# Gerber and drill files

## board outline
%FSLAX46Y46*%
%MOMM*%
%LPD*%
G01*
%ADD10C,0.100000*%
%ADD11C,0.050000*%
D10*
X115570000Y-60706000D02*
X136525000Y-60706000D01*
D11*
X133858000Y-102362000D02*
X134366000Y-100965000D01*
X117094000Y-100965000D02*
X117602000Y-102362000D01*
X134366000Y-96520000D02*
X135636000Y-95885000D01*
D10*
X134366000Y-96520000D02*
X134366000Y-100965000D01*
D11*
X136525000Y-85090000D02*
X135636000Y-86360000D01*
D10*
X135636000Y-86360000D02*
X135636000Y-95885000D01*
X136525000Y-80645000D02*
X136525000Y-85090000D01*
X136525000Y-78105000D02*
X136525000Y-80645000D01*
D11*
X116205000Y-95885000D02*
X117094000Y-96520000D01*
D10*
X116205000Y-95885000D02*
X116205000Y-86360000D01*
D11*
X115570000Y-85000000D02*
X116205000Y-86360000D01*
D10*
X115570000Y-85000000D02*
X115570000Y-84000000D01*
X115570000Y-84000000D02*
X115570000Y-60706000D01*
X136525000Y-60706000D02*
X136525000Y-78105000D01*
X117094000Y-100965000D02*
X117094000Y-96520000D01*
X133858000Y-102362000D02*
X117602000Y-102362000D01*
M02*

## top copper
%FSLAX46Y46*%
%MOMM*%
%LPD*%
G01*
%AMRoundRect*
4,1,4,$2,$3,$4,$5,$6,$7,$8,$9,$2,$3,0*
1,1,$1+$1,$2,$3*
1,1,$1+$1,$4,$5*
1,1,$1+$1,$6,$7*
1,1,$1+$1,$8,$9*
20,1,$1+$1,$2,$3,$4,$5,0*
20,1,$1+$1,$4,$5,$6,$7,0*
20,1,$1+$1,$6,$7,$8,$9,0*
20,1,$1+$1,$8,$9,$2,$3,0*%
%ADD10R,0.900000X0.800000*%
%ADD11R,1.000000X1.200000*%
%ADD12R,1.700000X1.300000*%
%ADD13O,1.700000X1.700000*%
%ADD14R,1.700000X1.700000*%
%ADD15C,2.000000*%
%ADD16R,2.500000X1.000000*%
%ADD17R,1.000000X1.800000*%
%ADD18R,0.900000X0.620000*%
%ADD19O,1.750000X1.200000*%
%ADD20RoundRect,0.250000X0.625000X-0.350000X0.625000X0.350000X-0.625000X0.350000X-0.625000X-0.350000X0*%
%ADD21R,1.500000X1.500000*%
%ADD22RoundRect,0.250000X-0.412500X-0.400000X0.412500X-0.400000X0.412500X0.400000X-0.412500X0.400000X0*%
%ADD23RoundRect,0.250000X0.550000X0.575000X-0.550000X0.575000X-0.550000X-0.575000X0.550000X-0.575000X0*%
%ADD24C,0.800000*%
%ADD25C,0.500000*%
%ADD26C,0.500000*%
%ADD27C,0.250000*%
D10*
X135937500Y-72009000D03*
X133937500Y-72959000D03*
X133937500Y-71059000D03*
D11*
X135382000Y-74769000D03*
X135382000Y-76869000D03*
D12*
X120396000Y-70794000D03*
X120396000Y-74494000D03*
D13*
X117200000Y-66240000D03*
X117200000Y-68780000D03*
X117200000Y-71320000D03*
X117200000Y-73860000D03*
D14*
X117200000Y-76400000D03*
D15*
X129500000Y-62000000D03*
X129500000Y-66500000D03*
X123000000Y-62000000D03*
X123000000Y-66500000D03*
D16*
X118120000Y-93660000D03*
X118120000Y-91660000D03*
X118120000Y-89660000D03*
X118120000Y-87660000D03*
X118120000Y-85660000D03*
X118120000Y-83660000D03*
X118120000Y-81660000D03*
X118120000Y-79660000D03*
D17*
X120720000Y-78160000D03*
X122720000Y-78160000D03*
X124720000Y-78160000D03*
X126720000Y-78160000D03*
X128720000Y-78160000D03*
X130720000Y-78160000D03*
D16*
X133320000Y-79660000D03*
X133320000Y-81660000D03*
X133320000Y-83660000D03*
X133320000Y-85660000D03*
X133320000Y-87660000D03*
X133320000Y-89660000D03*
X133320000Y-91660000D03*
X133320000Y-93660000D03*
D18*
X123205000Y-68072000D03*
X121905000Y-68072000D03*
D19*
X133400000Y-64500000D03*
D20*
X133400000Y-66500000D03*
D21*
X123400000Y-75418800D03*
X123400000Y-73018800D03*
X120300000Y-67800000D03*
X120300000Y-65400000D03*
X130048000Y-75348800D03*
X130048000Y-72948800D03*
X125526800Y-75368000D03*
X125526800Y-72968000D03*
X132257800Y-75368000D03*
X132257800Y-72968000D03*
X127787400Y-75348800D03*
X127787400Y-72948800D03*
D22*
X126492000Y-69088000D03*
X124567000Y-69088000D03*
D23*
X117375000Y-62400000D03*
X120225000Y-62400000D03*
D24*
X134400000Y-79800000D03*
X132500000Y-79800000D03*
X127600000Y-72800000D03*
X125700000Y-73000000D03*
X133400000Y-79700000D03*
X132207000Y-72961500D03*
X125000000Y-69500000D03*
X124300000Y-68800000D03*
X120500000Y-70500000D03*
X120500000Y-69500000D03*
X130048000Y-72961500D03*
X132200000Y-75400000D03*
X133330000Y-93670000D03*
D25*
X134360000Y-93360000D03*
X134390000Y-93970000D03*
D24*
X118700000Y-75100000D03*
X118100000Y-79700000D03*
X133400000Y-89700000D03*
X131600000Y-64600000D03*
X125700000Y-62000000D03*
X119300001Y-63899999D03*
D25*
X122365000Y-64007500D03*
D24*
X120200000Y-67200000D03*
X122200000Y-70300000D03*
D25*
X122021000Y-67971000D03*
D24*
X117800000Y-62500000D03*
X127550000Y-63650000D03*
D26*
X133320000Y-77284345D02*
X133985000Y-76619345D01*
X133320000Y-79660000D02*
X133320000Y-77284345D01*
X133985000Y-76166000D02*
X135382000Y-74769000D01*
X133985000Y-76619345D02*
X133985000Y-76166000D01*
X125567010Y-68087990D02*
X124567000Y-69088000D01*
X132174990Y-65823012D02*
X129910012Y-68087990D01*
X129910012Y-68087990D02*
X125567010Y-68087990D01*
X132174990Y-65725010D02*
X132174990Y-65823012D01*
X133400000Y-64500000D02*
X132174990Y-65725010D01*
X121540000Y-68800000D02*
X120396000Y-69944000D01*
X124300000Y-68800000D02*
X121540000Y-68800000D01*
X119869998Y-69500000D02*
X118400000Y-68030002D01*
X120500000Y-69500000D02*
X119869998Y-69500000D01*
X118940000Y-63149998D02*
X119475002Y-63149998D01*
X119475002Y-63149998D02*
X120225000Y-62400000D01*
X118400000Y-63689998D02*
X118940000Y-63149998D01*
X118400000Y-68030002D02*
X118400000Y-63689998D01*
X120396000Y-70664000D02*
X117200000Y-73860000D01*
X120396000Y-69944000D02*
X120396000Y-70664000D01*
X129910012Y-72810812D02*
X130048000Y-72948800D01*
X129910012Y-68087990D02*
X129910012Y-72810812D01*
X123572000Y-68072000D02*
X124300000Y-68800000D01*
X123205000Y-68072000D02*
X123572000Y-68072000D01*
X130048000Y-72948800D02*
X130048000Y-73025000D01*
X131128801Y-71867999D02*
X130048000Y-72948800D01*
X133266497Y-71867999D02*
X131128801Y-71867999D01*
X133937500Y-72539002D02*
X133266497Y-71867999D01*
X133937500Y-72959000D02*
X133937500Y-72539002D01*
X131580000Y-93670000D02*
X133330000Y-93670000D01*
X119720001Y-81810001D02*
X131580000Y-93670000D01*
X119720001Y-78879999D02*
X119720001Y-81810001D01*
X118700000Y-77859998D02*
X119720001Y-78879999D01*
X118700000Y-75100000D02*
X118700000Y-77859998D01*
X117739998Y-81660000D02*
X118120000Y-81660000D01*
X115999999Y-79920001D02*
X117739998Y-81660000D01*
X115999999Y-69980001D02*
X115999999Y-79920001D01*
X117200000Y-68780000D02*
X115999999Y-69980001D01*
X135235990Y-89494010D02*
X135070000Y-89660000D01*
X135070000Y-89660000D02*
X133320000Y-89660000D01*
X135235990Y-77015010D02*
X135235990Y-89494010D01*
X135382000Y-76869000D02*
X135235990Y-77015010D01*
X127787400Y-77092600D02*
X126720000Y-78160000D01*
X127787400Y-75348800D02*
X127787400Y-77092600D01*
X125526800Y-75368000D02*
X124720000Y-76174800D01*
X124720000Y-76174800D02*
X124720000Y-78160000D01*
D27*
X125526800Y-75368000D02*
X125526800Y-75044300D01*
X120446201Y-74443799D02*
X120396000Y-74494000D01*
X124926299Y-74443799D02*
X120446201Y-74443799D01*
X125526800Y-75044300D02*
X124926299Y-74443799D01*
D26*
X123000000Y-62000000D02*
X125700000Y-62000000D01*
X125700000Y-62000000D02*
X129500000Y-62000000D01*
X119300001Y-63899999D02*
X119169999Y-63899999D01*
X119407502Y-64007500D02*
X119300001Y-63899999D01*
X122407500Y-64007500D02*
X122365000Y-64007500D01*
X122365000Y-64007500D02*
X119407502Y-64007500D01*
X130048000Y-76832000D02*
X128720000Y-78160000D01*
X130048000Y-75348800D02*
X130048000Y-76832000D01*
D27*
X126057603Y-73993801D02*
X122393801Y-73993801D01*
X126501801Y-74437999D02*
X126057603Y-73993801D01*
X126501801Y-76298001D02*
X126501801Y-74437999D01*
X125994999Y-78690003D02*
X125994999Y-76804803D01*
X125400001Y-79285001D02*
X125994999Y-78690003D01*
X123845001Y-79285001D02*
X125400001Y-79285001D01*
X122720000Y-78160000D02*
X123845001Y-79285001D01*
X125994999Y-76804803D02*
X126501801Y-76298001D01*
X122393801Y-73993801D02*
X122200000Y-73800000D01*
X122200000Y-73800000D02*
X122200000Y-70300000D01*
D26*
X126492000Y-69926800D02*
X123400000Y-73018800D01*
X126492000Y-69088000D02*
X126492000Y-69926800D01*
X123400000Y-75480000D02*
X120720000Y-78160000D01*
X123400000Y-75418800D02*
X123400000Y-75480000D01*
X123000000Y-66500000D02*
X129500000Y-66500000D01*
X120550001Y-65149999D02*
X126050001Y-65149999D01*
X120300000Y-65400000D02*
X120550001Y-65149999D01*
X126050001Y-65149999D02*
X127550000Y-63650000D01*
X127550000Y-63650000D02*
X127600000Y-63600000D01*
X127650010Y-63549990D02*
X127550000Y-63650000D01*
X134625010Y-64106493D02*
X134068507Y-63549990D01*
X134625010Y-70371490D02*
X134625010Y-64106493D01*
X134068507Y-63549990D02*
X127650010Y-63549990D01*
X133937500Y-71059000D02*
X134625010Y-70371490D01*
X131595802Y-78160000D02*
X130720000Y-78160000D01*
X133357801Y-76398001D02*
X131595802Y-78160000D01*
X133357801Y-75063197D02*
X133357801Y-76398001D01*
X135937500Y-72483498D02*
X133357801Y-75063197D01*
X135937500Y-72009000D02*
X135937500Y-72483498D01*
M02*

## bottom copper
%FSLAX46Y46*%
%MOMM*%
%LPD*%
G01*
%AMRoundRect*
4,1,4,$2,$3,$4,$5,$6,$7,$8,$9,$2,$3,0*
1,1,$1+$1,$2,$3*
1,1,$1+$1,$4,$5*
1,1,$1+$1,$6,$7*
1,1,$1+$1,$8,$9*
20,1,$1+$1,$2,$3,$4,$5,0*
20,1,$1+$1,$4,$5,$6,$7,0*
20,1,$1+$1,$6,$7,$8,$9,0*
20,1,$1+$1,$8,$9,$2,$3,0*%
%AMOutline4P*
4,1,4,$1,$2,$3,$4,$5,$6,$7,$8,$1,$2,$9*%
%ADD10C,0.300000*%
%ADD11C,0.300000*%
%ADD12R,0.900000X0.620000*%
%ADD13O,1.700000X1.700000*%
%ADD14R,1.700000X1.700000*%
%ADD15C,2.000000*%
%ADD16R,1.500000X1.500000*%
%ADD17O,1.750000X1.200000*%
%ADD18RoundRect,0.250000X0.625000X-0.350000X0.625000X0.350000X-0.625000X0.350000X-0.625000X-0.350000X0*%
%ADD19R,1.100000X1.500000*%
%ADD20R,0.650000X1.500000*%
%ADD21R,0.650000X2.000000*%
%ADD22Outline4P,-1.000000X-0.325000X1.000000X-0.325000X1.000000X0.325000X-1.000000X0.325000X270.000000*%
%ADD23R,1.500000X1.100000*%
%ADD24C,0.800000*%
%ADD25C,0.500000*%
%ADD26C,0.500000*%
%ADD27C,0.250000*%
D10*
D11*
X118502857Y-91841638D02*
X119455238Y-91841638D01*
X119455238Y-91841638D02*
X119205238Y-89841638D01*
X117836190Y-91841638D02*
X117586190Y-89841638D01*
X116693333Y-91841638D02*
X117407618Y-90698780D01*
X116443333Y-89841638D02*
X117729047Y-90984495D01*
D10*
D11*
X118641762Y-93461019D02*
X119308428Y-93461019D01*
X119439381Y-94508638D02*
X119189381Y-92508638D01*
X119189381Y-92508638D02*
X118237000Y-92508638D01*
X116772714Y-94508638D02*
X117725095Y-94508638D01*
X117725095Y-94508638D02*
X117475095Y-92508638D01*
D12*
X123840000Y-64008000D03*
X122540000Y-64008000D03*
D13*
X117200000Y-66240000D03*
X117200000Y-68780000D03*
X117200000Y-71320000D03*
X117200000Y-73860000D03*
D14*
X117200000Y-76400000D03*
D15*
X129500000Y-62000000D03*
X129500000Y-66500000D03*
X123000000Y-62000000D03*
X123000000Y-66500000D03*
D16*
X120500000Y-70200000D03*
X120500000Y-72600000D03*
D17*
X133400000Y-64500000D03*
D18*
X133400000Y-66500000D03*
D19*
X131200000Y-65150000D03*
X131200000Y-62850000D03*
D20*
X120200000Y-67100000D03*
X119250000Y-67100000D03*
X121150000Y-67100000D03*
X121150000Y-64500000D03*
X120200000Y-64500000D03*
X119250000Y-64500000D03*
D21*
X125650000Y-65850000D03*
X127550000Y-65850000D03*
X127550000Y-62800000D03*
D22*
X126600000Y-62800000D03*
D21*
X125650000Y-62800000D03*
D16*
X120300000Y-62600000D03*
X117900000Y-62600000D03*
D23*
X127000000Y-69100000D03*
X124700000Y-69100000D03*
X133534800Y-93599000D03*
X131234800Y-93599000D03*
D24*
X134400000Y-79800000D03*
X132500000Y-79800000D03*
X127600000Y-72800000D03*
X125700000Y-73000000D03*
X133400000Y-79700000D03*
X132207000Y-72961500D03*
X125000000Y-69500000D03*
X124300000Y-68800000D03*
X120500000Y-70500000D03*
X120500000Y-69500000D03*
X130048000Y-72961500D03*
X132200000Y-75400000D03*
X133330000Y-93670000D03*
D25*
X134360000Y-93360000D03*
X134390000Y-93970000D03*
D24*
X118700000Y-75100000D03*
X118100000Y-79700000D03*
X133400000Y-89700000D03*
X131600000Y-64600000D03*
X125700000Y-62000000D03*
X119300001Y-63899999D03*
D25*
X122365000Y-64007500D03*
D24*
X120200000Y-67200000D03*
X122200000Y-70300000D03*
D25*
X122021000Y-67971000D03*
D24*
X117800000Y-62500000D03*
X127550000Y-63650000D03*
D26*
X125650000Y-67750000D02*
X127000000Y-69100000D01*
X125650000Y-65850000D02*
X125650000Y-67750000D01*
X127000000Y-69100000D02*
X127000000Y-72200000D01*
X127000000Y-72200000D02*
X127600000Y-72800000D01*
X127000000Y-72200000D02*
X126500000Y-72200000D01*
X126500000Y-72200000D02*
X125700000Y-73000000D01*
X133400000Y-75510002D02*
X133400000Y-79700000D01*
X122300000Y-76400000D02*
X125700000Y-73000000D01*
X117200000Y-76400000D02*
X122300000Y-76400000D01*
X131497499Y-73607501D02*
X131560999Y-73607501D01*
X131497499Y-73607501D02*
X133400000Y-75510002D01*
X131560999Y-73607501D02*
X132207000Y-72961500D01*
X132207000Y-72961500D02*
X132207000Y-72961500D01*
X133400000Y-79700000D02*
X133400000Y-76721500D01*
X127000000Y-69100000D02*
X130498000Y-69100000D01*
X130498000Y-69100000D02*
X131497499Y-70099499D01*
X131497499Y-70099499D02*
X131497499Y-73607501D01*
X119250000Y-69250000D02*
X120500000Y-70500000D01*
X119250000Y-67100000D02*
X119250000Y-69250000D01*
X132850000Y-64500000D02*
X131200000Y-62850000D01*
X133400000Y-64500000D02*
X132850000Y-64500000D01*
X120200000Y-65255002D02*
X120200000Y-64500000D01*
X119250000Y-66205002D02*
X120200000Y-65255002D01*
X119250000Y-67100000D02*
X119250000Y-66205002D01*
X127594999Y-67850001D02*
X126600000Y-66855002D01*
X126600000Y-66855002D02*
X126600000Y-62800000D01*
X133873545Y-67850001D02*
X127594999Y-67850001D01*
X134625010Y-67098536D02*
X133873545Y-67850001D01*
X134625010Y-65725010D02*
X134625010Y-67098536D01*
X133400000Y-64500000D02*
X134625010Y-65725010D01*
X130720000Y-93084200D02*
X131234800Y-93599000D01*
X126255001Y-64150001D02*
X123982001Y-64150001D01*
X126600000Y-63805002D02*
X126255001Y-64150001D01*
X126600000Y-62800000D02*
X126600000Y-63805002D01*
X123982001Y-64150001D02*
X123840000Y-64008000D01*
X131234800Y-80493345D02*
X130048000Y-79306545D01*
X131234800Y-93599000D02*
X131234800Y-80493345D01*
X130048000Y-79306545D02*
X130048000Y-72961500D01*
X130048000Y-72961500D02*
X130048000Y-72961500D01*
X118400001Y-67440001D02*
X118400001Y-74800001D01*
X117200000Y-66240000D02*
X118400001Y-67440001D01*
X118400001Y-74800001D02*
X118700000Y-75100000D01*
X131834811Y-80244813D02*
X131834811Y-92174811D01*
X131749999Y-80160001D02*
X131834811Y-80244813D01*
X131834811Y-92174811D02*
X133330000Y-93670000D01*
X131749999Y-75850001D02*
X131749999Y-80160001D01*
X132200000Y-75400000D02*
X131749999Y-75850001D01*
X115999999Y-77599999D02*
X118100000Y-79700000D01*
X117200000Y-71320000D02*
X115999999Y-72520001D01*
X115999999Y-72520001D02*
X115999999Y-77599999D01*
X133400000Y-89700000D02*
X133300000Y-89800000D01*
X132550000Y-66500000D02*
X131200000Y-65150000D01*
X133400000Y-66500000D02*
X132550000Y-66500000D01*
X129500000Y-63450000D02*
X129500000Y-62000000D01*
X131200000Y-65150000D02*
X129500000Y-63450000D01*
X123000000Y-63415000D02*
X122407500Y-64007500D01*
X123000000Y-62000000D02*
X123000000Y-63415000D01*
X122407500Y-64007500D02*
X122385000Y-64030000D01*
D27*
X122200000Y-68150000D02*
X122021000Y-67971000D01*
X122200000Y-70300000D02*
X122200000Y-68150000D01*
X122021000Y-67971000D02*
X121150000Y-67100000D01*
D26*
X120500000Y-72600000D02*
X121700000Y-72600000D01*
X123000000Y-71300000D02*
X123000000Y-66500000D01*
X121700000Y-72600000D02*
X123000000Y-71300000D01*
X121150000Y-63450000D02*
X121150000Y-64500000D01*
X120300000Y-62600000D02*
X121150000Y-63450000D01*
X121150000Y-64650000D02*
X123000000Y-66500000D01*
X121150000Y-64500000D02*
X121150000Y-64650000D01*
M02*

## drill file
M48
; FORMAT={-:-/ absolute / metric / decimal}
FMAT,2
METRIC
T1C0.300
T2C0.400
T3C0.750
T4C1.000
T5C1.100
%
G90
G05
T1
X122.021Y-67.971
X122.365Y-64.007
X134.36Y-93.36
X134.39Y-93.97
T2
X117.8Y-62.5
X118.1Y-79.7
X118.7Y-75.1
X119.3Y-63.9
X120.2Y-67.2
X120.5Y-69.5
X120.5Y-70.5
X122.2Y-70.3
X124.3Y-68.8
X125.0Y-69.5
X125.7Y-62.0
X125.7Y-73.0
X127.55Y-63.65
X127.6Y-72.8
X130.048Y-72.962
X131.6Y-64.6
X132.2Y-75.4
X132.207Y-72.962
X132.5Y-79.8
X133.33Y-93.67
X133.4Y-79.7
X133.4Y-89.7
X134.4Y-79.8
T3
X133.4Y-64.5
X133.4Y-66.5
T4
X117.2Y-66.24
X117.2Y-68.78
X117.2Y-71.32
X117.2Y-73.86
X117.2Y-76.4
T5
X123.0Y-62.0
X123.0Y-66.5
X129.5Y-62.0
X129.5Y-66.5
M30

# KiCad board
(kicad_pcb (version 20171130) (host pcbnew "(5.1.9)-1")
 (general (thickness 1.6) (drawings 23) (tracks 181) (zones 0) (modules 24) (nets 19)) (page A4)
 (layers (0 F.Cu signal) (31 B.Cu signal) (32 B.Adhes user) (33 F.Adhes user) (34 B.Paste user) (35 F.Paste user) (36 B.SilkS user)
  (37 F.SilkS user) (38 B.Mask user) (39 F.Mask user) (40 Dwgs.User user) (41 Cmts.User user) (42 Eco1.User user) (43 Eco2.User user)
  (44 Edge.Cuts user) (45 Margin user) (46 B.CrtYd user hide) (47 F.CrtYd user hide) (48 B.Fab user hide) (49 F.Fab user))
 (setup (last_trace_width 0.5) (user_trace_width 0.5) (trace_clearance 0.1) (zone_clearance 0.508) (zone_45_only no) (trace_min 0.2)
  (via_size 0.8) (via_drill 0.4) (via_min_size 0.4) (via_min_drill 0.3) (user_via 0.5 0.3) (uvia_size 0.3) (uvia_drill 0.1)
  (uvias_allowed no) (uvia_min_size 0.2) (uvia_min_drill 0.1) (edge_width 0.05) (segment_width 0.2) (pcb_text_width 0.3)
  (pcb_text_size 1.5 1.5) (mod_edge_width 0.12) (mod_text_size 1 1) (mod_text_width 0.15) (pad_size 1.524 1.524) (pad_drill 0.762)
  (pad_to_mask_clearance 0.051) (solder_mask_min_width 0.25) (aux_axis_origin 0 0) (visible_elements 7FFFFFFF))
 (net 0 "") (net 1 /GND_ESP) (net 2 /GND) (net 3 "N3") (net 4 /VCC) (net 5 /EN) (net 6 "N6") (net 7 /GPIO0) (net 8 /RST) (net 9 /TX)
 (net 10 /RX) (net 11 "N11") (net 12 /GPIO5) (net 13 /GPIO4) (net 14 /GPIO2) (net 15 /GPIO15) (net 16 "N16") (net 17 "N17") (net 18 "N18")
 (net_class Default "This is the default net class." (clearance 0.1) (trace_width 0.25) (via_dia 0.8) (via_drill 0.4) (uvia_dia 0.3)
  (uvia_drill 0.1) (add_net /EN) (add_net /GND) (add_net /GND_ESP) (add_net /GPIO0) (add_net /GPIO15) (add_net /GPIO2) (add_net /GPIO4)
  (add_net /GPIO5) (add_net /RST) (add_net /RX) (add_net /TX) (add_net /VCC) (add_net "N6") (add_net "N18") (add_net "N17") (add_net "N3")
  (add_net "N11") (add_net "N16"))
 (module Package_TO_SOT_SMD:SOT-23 (layer F.Cu) (at 134.9375 72.009)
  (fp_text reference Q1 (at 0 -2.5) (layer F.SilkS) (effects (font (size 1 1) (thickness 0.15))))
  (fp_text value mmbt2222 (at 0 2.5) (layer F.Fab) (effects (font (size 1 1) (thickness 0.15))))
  (pad 3 smd rect (at 1 0) (size 0.9 0.8) (layers F.Cu F.Paste F.Mask) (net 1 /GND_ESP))
  (pad 2 smd rect (at -1 0.95) (size 0.9 0.8) (layers F.Cu F.Paste F.Mask) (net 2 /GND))
  (pad 1 smd rect (at -1 -0.95) (size 0.9 0.8) (layers F.Cu F.Paste F.Mask) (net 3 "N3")))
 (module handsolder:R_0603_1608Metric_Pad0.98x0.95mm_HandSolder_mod (layer F.Cu) (at 135.382 75.819 90)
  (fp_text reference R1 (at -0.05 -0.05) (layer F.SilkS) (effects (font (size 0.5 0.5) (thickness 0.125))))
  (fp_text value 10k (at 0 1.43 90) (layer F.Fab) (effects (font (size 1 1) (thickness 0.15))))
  (pad 2 smd rect (at 1.05 0 90) (size 1.2 1) (layers F.Cu F.Paste F.Mask) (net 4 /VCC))
  (pad 1 smd rect (at -1.05 0 90) (size 1.2 1) (layers F.Cu F.Paste F.Mask) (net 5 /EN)))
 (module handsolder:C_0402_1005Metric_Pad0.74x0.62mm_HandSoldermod (layer B.Cu) (at 123.19 64.008)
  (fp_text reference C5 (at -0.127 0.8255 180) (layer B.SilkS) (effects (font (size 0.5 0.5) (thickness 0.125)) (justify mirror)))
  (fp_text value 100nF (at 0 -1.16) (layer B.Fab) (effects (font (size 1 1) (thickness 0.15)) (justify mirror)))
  (pad 2 smd rect (at 0.65 0) (size 0.9 0.62) (layers B.Cu B.Paste B.Mask) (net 2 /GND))
  (pad 1 smd rect (at -0.65 0) (size 0.9 0.62) (layers B.Cu B.Paste B.Mask) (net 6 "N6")))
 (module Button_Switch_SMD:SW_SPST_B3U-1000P (layer F.Cu) (at 120.396 72.644 90)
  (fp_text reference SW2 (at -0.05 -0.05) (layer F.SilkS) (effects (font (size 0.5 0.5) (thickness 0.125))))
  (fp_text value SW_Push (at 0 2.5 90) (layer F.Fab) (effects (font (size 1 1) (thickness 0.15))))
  (pad 2 smd rect (at 1.85 0 90) (size 1.3 1.7) (layers F.Cu F.Paste F.Mask) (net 2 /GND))
  (pad 1 smd rect (at -1.85 0 90) (size 1.3 1.7) (layers F.Cu F.Paste F.Mask) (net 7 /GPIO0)))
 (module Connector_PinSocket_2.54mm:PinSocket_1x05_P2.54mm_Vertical (layer F.Cu) (at 117.2 76.4 180)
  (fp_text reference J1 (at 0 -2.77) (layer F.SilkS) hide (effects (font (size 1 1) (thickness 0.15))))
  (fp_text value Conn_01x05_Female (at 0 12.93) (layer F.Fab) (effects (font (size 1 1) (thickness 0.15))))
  (pad 5 thru_hole oval (at 0 10.16 180) (size 1.7 1.7) (drill 1) (layers *.Cu *.Mask) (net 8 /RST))
  (pad 4 thru_hole oval (at 0 7.62 180) (size 1.7 1.7) (drill 1) (layers *.Cu *.Mask) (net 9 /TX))
  (pad 3 thru_hole oval (at 0 5.08 180) (size 1.7 1.7) (drill 1) (layers *.Cu *.Mask) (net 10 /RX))
  (pad 2 thru_hole oval (at 0 2.54 180) (size 1.7 1.7) (drill 1) (layers *.Cu *.Mask) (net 2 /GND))
  (pad 1 thru_hole rect (at 0 0 180) (size 1.7 1.7) (drill 1) (layers *.Cu *.Mask) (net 4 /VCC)))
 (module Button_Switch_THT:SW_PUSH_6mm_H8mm (layer F.Cu) (at 123 62)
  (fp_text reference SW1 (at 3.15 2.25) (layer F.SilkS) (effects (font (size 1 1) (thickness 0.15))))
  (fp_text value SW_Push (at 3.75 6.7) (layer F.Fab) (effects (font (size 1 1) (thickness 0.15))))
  (pad 1 thru_hole circle (at 6.5 0 90) (size 2 2) (drill 1.1) (layers *.Cu *.Mask) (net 6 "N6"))
  (pad 2 thru_hole circle (at 6.5 4.5 90) (size 2 2) (drill 1.1) (layers *.Cu *.Mask) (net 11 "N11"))
  (pad 1 thru_hole circle (at 0 0 90) (size 2 2) (drill 1.1) (layers *.Cu *.Mask) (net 6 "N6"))
  (pad 2 thru_hole circle (at 0 4.5 90) (size 2 2) (drill 1.1) (layers *.Cu *.Mask) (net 11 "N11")))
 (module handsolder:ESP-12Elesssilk (layer F.Cu) (at 125.72 90.16 180)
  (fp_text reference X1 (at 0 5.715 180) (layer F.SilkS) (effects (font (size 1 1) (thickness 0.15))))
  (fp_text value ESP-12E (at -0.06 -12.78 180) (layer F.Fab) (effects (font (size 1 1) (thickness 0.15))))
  (pad 22 smd rect (at 7.6 -3.5 180) (size 2.5 1) (layers F.Cu F.Paste F.Mask))
  (pad 21 smd rect (at 7.6 -1.5 180) (size 2.5 1) (layers F.Cu F.Paste F.Mask))
  (pad 20 smd rect (at 7.6 0.5 180) (size 2.5 1) (layers F.Cu F.Paste F.Mask))
  (pad 19 smd rect (at 7.6 2.5 180) (size 2.5 1) (layers F.Cu F.Paste F.Mask))
  (pad 18 smd rect (at 7.6 4.5 180) (size 2.5 1) (layers F.Cu F.Paste F.Mask))
  (pad 17 smd rect (at 7.6 6.5 180) (size 2.5 1) (layers F.Cu F.Paste F.Mask))
  (pad 16 smd rect (at 7.6 8.5 180) (size 2.5 1) (layers F.Cu F.Paste F.Mask) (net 9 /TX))
  (pad 15 smd rect (at 7.6 10.5 180) (size 2.5 1) (layers F.Cu F.Paste F.Mask) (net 10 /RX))
  (pad 14 smd rect (at 5 12 180) (size 1 1.8) (layers F.Cu F.Paste F.Mask) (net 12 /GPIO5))
  (pad 13 smd rect (at 3 12 180) (size 1 1.8) (layers F.Cu F.Paste F.Mask) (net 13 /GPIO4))
  (pad 12 smd rect (at 1 12 180) (size 1 1.8) (layers F.Cu F.Paste F.Mask) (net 7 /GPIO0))
  (pad 11 smd rect (at -1 12 180) (size 1 1.8) (layers F.Cu F.Paste F.Mask) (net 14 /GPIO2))
  (pad 10 smd rect (at -3 12 180) (size 1 1.8) (layers F.Cu F.Paste F.Mask) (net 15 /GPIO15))
  (pad 9 smd rect (at -5 12 180) (size 1 1.8) (layers F.Cu F.Paste F.Mask) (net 1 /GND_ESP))
  (pad 8 smd rect (at -7.6 10.5 180) (size 2.5 1) (layers F.Cu F.Paste F.Mask) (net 4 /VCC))
  (pad 7 smd rect (at -7.6 8.5 180) (size 2.5 1) (layers F.Cu F.Paste F.Mask))
  (pad 6 smd rect (at -7.6 6.5 180) (size 2.5 1) (layers F.Cu F.Paste F.Mask))
  (pad 5 smd rect (at -7.6 4.5 180) (size 2.5 1) (layers F.Cu F.Paste F.Mask))
  (pad 4 smd rect (at -7.6 2.5 180) (size 2.5 1) (layers F.Cu F.Paste F.Mask))
  (pad 3 smd rect (at -7.6 0.5 180) (size 2.5 1) (layers F.Cu F.Paste F.Mask) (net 5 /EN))
  (pad 2 smd rect (at -7.6 -1.5 180) (size 2.5 1) (layers F.Cu F.Paste F.Mask))
  (pad 1 smd rect (at -7.6 -3.5 180) (size 2.5 1) (layers F.Cu F.Paste F.Mask) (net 8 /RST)))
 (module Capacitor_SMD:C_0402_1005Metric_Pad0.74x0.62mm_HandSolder (layer F.Cu) (at 122.555 68.072)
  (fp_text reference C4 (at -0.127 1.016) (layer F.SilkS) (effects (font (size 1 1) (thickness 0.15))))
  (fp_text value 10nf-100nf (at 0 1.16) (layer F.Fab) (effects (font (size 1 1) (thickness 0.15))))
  (pad 2 smd rect (at 0.65 0) (size 0.9 0.62) (layers F.Cu F.Paste F.Mask) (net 2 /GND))
  (pad 1 smd rect (at -0.65 0) (size 0.9 0.62) (layers F.Cu F.Paste F.Mask) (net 13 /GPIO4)))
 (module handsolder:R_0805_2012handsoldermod (layer B.Cu) (at 120.5 71.4 90)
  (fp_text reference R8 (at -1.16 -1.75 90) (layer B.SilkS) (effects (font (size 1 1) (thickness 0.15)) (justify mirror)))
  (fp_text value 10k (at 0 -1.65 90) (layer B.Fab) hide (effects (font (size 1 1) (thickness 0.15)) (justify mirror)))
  (pad 2 smd rect (at 1.2 0 90) (size 1.5 1.5) (layers B.Cu B.Paste B.Mask) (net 2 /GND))
  (pad 1 smd rect (at -1.2 0 90) (size 1.5 1.5) (layers B.Cu B.Paste B.Mask) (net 11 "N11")))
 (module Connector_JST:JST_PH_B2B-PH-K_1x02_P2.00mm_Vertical (layer F.Cu) (at 133.4 66.5 90)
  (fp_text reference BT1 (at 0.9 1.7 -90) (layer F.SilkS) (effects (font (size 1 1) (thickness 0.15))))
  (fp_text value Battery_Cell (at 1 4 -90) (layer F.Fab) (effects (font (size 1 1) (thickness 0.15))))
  (pad 2 thru_hole oval (at 2 0 90) (size 1.2 1.75) (drill 0.75) (layers *.Cu *.Mask) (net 2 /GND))
  (pad 1 thru_hole roundrect (at 0 0 90) (size 1.2 1.75) (drill 0.75) (layers *.Cu *.Mask) (roundrect_rratio 0.208333) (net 6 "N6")))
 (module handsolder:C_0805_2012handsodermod (layer B.Cu) (at 131.2 64 270)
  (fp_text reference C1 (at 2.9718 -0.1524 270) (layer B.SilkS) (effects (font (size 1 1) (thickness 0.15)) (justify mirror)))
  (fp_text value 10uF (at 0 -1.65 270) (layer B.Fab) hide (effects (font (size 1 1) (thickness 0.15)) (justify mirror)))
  (pad 2 smd rect (at 1.15 0 270) (size 1.5 1.1) (layers B.Cu B.Paste B.Mask) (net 6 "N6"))
  (pad 1 smd rect (at -1.15 0 270) (size 1.5 1.1) (layers B.Cu B.Paste B.Mask) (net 2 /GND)))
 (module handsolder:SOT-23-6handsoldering (layer B.Cu) (at 120.2 65.8 270)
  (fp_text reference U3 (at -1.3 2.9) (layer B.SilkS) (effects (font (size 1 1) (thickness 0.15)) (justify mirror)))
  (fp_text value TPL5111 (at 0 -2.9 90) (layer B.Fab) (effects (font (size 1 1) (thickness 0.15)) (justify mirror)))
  (pad 5 smd rect (at 1.3 0 270) (size 1.5 0.65) (layers B.Cu B.Paste B.Mask) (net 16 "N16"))
  (pad 6 smd rect (at 1.3 0.95 270) (size 1.5 0.65) (layers B.Cu B.Paste B.Mask) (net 2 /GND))
  (pad 4 smd rect (at 1.3 -0.95 270) (size 1.5 0.65) (layers B.Cu B.Paste B.Mask) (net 13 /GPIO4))
  (pad 3 smd rect (at -1.3 -0.95 270) (size 1.5 0.65) (layers B.Cu B.Paste B.Mask) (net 11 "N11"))
  (pad 2 smd rect (at -1.3 0 270) (size 1.5 0.65) (layers B.Cu B.Paste B.Mask) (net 2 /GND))
  (pad 1 smd rect (at -1.3 0.95 270) (size 1.5 0.65) (layers B.Cu B.Paste B.Mask) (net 6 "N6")))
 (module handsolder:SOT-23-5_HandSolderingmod (layer B.Cu) (at 126.6 64.35 270)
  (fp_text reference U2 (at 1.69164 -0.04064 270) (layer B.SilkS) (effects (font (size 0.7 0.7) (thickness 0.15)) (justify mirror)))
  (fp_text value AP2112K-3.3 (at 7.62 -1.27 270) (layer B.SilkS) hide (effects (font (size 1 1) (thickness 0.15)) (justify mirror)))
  (pad 5 smd rect (at 1.5 0.95 270) (size 2 0.65) (layers B.Cu B.Paste B.Mask) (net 4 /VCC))
  (pad 4 smd rect (at 1.5 -0.95 270) (size 2 0.65) (layers B.Cu B.Paste B.Mask))
  (pad 3 smd rect (at -1.55 -0.95 270) (size 2 0.65) (layers B.Cu B.Paste B.Mask) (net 3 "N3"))
  (pad 2 smd trapezoid (at -1.55 0 270) (size 2 0.65) (layers B.Cu B.Paste B.Mask) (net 2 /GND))
  (pad 1 smd rect (at -1.55 0.95 270) (size 2 0.65) (layers B.Cu B.Paste B.Mask) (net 6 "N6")))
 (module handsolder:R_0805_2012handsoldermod (layer F.Cu) (at 123.4 74.2188 270)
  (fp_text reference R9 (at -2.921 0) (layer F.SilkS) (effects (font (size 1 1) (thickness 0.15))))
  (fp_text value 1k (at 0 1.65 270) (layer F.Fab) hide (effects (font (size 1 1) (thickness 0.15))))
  (pad 2 smd rect (at 1.2 0 270) (size 1.5 1.5) (layers F.Cu F.Paste F.Mask) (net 12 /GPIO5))
  (pad 1 smd rect (at -1.2 0 270) (size 1.5 1.5) (layers F.Cu F.Paste F.Mask) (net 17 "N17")))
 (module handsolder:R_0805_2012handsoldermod (layer F.Cu) (at 120.3 66.6 270)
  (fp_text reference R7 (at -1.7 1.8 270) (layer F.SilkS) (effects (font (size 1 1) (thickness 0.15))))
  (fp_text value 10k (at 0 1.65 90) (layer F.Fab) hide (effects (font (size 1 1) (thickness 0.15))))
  (pad 2 smd rect (at 1.2 0 270) (size 1.5 1.5) (layers F.Cu F.Paste F.Mask) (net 16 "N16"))
  (pad 1 smd rect (at -1.2 0 270) (size 1.5 1.5) (layers F.Cu F.Paste F.Mask) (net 3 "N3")))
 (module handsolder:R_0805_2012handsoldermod (layer B.Cu) (at 119.1 62.6)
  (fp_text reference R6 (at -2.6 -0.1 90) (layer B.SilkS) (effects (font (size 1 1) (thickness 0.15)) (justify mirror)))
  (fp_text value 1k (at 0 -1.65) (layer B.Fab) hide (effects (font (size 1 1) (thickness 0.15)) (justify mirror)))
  (pad 2 smd rect (at 1.2 0) (size 1.5 1.5) (layers B.Cu B.Paste B.Mask) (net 11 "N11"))
  (pad 1 smd rect (at -1.2 0) (size 1.5 1.5) (layers B.Cu B.Paste B.Mask) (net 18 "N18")))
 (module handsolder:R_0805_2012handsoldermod (layer F.Cu) (at 130.048 74.1488 270)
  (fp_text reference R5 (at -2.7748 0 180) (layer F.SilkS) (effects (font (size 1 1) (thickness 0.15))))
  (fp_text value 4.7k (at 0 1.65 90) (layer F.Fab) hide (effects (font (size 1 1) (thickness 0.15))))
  (pad 2 smd rect (at 1.2 0 270) (size 1.5 1.5) (layers F.Cu F.Paste F.Mask) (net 15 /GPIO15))
  (pad 1 smd rect (at -1.2 0 270) (size 1.5 1.5) (layers F.Cu F.Paste F.Mask) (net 2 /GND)))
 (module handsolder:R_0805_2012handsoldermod (layer F.Cu) (at 125.5268 74.168 270)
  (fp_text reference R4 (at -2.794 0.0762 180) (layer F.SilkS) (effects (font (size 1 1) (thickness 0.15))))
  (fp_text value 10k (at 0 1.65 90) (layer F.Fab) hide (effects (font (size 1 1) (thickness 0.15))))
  (pad 2 smd rect (at 1.2 0 270) (size 1.5 1.5) (layers F.Cu F.Paste F.Mask) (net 7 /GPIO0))
  (pad 1 smd rect (at -1.2 0 270) (size 1.5 1.5) (layers F.Cu F.Paste F.Mask) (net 4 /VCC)))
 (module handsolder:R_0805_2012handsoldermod (layer F.Cu) (at 132.2578 74.168 270)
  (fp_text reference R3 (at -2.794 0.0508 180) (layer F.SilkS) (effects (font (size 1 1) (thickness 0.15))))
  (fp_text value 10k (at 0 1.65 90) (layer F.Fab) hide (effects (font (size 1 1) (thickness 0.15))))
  (pad 2 smd rect (at 1.2 0 270) (size 1.5 1.5) (layers F.Cu F.Paste F.Mask) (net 8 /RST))
  (pad 1 smd rect (at -1.2 0 270) (size 1.5 1.5) (layers F.Cu F.Paste F.Mask) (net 4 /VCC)))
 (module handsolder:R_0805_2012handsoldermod (layer F.Cu) (at 127.7874 74.1488 270)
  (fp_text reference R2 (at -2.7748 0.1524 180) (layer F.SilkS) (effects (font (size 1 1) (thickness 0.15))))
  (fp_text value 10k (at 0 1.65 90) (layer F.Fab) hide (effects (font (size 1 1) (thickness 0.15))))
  (pad 2 smd rect (at 1.2 0 270) (size 1.5 1.5) (layers F.Cu F.Paste F.Mask) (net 14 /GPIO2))
  (pad 1 smd rect (at -1.2 0 270) (size 1.5 1.5) (layers F.Cu F.Paste F.Mask) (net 4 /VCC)))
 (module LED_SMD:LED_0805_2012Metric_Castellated (layer F.Cu) (at 125.5295 69.088)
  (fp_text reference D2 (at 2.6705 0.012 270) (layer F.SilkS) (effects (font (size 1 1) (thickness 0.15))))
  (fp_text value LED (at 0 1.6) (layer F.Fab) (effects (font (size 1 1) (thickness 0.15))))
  (pad 2 smd roundrect (at 0.9625 0) (size 1.325 1.3) (layers F.Cu F.Paste F.Mask) (roundrect_rratio 0.1923076923076923) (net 17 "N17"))
  (pad 1 smd roundrect (at -0.9625 0) (size 1.325 1.3) (layers F.Cu F.Paste F.Mask) (roundrect_rratio 0.1923076923076923) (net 2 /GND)))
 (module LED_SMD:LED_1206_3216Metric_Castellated (layer F.Cu) (at 118.8 62.4 180)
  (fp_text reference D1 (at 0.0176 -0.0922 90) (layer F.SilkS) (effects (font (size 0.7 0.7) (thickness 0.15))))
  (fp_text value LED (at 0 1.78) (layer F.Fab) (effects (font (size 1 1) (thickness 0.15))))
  (pad 2 smd roundrect (at 1.425 0 180) (size 1.6 1.65) (layers F.Cu F.Paste F.Mask) (roundrect_rratio 0.15625) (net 18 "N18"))
  (pad 1 smd roundrect (at -1.425 0 180) (size 1.6 1.65) (layers F.Cu F.Paste F.Mask) (roundrect_rratio 0.15625) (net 2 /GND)))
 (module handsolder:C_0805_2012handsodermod (layer B.Cu) (at 125.85 69.1)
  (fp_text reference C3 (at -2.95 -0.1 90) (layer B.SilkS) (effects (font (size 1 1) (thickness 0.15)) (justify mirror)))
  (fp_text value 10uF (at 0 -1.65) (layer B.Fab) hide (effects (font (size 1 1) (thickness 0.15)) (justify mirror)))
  (pad 2 smd rect (at 1.15 0) (size 1.5 1.1) (layers B.Cu B.Paste B.Mask) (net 4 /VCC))
  (pad 1 smd rect (at -1.15 0) (size 1.5 1.1) (layers B.Cu B.Paste B.Mask) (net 2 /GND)))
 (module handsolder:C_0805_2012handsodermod (layer B.Cu) (at 132.3848 93.599)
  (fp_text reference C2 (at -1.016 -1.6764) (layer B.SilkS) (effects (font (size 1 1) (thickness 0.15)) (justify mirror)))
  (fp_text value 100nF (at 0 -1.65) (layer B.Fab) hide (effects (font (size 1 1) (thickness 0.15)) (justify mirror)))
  (pad 2 smd rect (at 1.15 0) (size 1.5 1.1) (layers B.Cu B.Paste B.Mask) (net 8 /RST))
  (pad 1 smd rect (at -1.15 0) (size 1.5 1.1) (layers B.Cu B.Paste B.Mask) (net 2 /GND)))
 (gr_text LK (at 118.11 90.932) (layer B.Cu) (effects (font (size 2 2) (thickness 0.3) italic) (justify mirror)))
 (gr_line (start 115.57 60.706) (end 136.525 60.706) (layer Edge.Cuts) (width 0.1))
 (gr_line (start 133.858 102.362) (end 134.366 100.965) (layer Edge.Cuts) (width 0.05))
 (gr_line (start 117.094 100.965) (end 117.602 102.362) (layer Edge.Cuts) (width 0.05))
 (gr_line (start 134.366 96.52) (end 135.636 95.885) (layer Edge.Cuts) (width 0.05))
 (gr_line (start 134.366 96.52) (end 134.366 100.965) (layer Edge.Cuts) (width 0.1))
 (gr_line (start 136.525 85.09) (end 135.636 86.36) (layer Edge.Cuts) (width 0.05))
 (gr_line (start 135.636 86.36) (end 135.636 95.885) (layer Edge.Cuts) (width 0.1))
 (gr_line (start 136.525 80.645) (end 136.525 85.09) (layer Edge.Cuts) (width 0.1))
 (gr_line (start 136.525 78.105) (end 136.525 80.645) (layer Edge.Cuts) (width 0.1))
 (gr_line (start 116.205 95.885) (end 117.094 96.52) (layer Edge.Cuts) (width 0.05))
 (gr_line (start 116.205 95.885) (end 116.205 86.36) (layer Edge.Cuts) (width 0.1))
 (gr_line (start 115.57 85) (end 116.205 86.36) (layer Edge.Cuts) (width 0.05))
 (gr_line (start 115.57 85) (end 115.57 84) (layer Edge.Cuts) (width 0.1))
 (gr_line (start 115.57 84) (end 115.57 60.706) (layer Edge.Cuts) (width 0.1))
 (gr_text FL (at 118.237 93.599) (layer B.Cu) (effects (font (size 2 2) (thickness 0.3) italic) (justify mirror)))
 (gr_line (start 136.525 60.706) (end 136.525 78.105) (layer Edge.Cuts) (width 0.1))
 (gr_line (start 117.094 100.965) (end 117.094 96.52) (layer Edge.Cuts) (width 0.1))
 (gr_line (start 133.858 102.362) (end 117.602 102.362) (layer Edge.Cuts) (width 0.1))
 (via (at 134.4 79.8) (size 0.8) (drill 0.4) (layers F.Cu B.Cu) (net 4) (status 30))
 (via (at 132.5 79.8) (size 0.8) (drill 0.4) (layers F.Cu B.Cu) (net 4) (status 30))
 (segment (start 125.65 67.75) (end 127 69.1) (width 0.5) (layer B.Cu) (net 4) (status 20))
 (segment (start 125.65 65.85) (end 125.65 67.75) (width 0.5) (layer B.Cu) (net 4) (status 10))
 (segment (start 127 69.1) (end 127 72.2) (width 0.5) (layer B.Cu) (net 4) (status 10))
 (segment (start 127 72.2) (end 127.6 72.8) (width 0.5) (layer B.Cu) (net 4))
 (segment (start 127 72.2) (end 126.5 72.2) (width 0.5) (layer B.Cu) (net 4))
 (segment (start 126.5 72.2) (end 125.7 73) (width 0.5) (layer B.Cu) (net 4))
 (via (at 127.6 72.8) (size 0.8) (drill 0.4) (layers F.Cu B.Cu) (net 4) (status 30))
 (via (at 125.7 73) (size 0.8) (drill 0.4) (layers F.Cu B.Cu) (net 4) (status 30))
 (segment (start 133.4 75.510002) (end 133.4 79.7) (width 0.5) (layer B.Cu) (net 4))
 (via (at 133.4 79.7) (size 0.8) (drill 0.4) (layers F.Cu B.Cu) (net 4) (status 30))
 (segment (start 122.3 76.4) (end 125.7 73) (width 0.5) (layer B.Cu) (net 4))
 (segment (start 117.2 76.4) (end 122.3 76.4) (width 0.5) (layer B.Cu) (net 4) (status 10))
 (segment (start 131.497499 73.607501) (end 131.560999 73.607501) (width 0.5) (layer B.Cu) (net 4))
 (segment (start 131.497499 73.607501) (end 133.4 75.510002) (width 0.5) (layer B.Cu) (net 4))
 (segment (start 131.560999 73.607501) (end 132.207 72.9615) (width 0.5) (layer B.Cu) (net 4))
 (segment (start 132.207 72.9615) (end 132.207 72.9615) (width 0.5) (layer B.Cu) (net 4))
 (via (at 132.207 72.9615) (size 0.8) (drill 0.4) (layers F.Cu B.Cu) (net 4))
 (segment (start 133.4 79.7) (end 133.4 76.7215) (width 0.5) (layer B.Cu) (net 4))
 (segment (start 133.32 77.284345) (end 133.985 76.619345) (width 0.5) (layer F.Cu) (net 4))
 (segment (start 133.32 79.66) (end 133.32 77.284345) (width 0.5) (layer F.Cu) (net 4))
 (segment (start 133.985 76.166) (end 135.382 74.769) (width 0.5) (layer F.Cu) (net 4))
 (segment (start 133.985 76.619345) (end 133.985 76.166) (width 0.5) (layer F.Cu) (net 4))
 (segment (start 127 69.1) (end 130.498 69.1) (width 0.5) (layer B.Cu) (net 4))
 (segment (start 130.498 69.1) (end 131.497499 70.099499) (width 0.5) (layer B.Cu) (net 4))
 (segment (start 131.497499 70.099499) (end 131.497499 73.607501) (width 0.5) (layer B.Cu) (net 4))
 (via (at 125 69.5) (size 0.8) (drill 0.4) (layers F.Cu B.Cu) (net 2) (status 30))
 (via (at 124.3 68.8) (size 0.8) (drill 0.4) (layers F.Cu B.Cu) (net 2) (status 30))
 (via (at 120.5 70.5) (size 0.8) (drill 0.4) (layers F.Cu B.Cu) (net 2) (status 30))
 (via (at 120.5 69.5) (size 0.8) (drill 0.4) (layers F.Cu B.Cu) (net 2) (status 30))
 (segment (start 119.25 69.25) (end 120.5 70.5) (width 0.5) (layer B.Cu) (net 2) (status 20))
 (segment (start 119.25 67.1) (end 119.25 69.25) (width 0.5) (layer B.Cu) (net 2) (status 10))
 (segment (start 132.85 64.5) (end 131.2 62.85) (width 0.5) (layer B.Cu) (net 2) (status 30))
 (segment (start 133.4 64.5) (end 132.85 64.5) (width 0.5) (layer B.Cu) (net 2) (status 30))
 (segment (start 120.2 65.255002) (end 120.2 64.5) (width 0.5) (layer B.Cu) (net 2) (status 20))
 (segment (start 119.25 66.205002) (end 120.2 65.255002) (width 0.5) (layer B.Cu) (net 2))
 (segment (start 119.25 67.1) (end 119.25 66.205002) (width 0.5) (layer B.Cu) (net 2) (status 10))
 (segment (start 127.594999 67.850001) (end 126.6 66.855002) (width 0.5) (layer B.Cu) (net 2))
 (segment (start 126.6 66.855002) (end 126.6 62.8) (width 0.5) (layer B.Cu) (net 2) (status 20))
 (segment (start 133.873545 67.850001) (end 127.594999 67.850001) (width 0.5) (layer B.Cu) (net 2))
 (segment (start 134.62501 67.098536) (end 133.873545 67.850001) (width 0.5) (layer B.Cu) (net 2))
 (segment (start 134.62501 65.72501) (end 134.62501 67.098536) (width 0.5) (layer B.Cu) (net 2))
 (segment (start 133.4 64.5) (end 134.62501 65.72501) (width 0.5) (layer B.Cu) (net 2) (status 10))
 (segment (start 125.56701 68.08799) (end 124.567 69.088) (width 0.5) (layer F.Cu) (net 2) (status 20))
 (segment (start 132.17499 65.823012) (end 129.910012 68.08799) (width 0.5) (layer F.Cu) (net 2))
 (segment (start 129.910012 68.08799) (end 125.56701 68.08799) (width 0.5) (layer F.Cu) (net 2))
 (segment (start 132.17499 65.72501) (end 132.17499 65.823012) (width 0.5) (layer F.Cu) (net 2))
 (segment (start 133.4 64.5) (end 132.17499 65.72501) (width 0.5) (layer F.Cu) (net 2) (status 10))
 (segment (start 121.54 68.8) (end 120.396 69.944) (width 0.5) (layer F.Cu) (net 2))
 (segment (start 124.3 68.8) (end 121.54 68.8) (width 0.5) (layer F.Cu) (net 2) (status 10))
 (segment (start 119.869998 69.5) (end 118.4 68.030002) (width 0.5) (layer F.Cu) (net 2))
 (segment (start 120.5 69.5) (end 119.869998 69.5) (width 0.5) (layer F.Cu) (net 2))
 (segment (start 118.94 63.149998) (end 119.475002 63.149998) (width 0.5) (layer F.Cu) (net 2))
 (segment (start 119.475002 63.149998) (end 120.225 62.4) (width 0.5) (layer F.Cu) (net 2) (status 20))
 (segment (start 118.4 63.689998) (end 118.94 63.149998) (width 0.5) (layer F.Cu) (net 2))
 (segment (start 118.4 68.030002) (end 118.4 63.689998) (width 0.5) (layer F.Cu) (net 2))
 (segment (start 120.396 70.664) (end 117.2 73.86) (width 0.5) (layer F.Cu) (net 2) (status 30))
 (segment (start 120.396 69.944) (end 120.396 70.664) (width 0.5) (layer F.Cu) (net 2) (status 20))
 (segment (start 129.910012 72.810812) (end 130.048 72.9488) (width 0.5) (layer F.Cu) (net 2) (status 30))
 (segment (start 129.910012 68.08799) (end 129.910012 72.810812) (width 0.5) (layer F.Cu) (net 2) (status 20))
 (segment (start 130.72 93.0842) (end 131.2348 93.599) (width 0.5) (layer B.Cu) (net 2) (status 30))
 (segment (start 123.572 68.072) (end 124.3 68.8) (width 0.5) (layer F.Cu) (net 2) (status 30))
 (segment (start 123.205 68.072) (end 123.572 68.072) (width 0.5) (layer F.Cu) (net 2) (status 30))
 (segment (start 126.255001 64.150001) (end 123.982001 64.150001) (width 0.5) (layer B.Cu) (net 2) (status 20))
 (segment (start 126.6 63.805002) (end 126.255001 64.150001) (width 0.5) (layer B.Cu) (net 2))
 (segment (start 126.6 62.8) (end 126.6 63.805002) (width 0.5) (layer B.Cu) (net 2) (status 10))
 (segment (start 123.982001 64.150001) (end 123.84 64.008) (width 0.5) (layer B.Cu) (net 2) (status 30))
 (segment (start 130.048 72.9488) (end 130.048 73.025) (width 0.5) (layer F.Cu) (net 2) (status 30))
 (segment (start 131.128801 71.867999) (end 130.048 72.9488) (width 0.5) (layer F.Cu) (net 2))
 (segment (start 133.266497 71.867999) (end 131.128801 71.867999) (width 0.5) (layer F.Cu) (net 2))
 (segment (start 133.9375 72.539002) (end 133.266497 71.867999) (width 0.5) (layer F.Cu) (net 2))
 (segment (start 133.9375 72.959) (end 133.9375 72.539002) (width 0.5) (layer F.Cu) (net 2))
 (segment (start 131.2348 80.493345) (end 130.048 79.306545) (width 0.5) (layer B.Cu) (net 2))
 (segment (start 131.2348 93.599) (end 131.2348 80.493345) (width 0.5) (layer B.Cu) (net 2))
 (segment (start 130.048 79.306545) (end 130.048 72.9615) (width 0.5) (layer B.Cu) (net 2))
 (segment (start 130.048 72.9615) (end 130.048 72.9615) (width 0.5) (layer B.Cu) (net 2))
 (via (at 130.048 72.9615) (size 0.8) (drill 0.4) (layers F.Cu B.Cu) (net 2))
 (via (at 132.2 75.4) (size 0.8) (drill 0.4) (layers F.Cu B.Cu) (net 8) (status 30))
 (via (at 133.33 93.67) (size 0.8) (drill 0.4) (layers F.Cu B.Cu) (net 8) (status 30))
 (via (at 134.36 93.36) (size 0.5) (drill 0.3) (layers F.Cu B.Cu) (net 8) (status 30))
 (via (at 134.39 93.97) (size 0.5) (drill 0.3) (layers F.Cu B.Cu) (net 8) (status 30))
 (segment (start 118.400001 67.440001) (end 118.400001 74.800001) (width 0.5) (layer B.Cu) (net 8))
 (segment (start 117.2 66.24) (end 118.400001 67.440001) (width 0.5) (layer B.Cu) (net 8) (status 10))
 (segment (start 118.400001 74.800001) (end 118.7 75.1) (width 0.5) (layer B.Cu) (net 8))
 (via (at 118.7 75.1) (size 0.8) (drill 0.4) (layers F.Cu B.Cu) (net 8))
 (segment (start 131.58 93.67) (end 133.33 93.67) (width 0.5) (layer F.Cu) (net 8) (status 20))
 (segment (start 119.720001 81.810001) (end 131.58 93.67) (width 0.5) (layer F.Cu) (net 8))
 (segment (start 119.720001 78.879999) (end 119.720001 81.810001) (width 0.5) (layer F.Cu) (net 8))
 (segment (start 118.7 77.859998) (end 119.720001 78.879999) (width 0.5) (layer F.Cu) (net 8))
 (segment (start 118.7 75.1) (end 118.7 77.859998) (width 0.5) (layer F.Cu) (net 8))
 (segment (start 131.834811 80.244813) (end 131.834811 92.174811) (width 0.5) (layer B.Cu) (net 8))
 (segment (start 131.749999 80.160001) (end 131.834811 80.244813) (width 0.5) (layer B.Cu) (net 8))
 (segment (start 131.834811 92.174811) (end 133.33 93.67) (width 0.5) (layer B.Cu) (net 8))
 (segment (start 131.749999 75.850001) (end 131.749999 80.160001) (width 0.5) (layer B.Cu) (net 8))
 (segment (start 132.2 75.4) (end 131.749999 75.850001) (width 0.5) (layer B.Cu) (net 8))
 (via (at 118.1 79.7) (size 0.8) (drill 0.4) (layers F.Cu B.Cu) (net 10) (status 30))
 (segment (start 115.999999 77.599999) (end 118.1 79.7) (width 0.5) (layer B.Cu) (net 10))
 (segment (start 117.2 71.32) (end 115.999999 72.520001) (width 0.5) (layer B.Cu) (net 10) (status 10))
 (segment (start 115.999999 72.520001) (end 115.999999 77.599999) (width 0.5) (layer B.Cu) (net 10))
 (segment (start 117.739998 81.66) (end 118.12 81.66) (width 0.5) (layer F.Cu) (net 9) (status 30))
 (segment (start 115.999999 79.920001) (end 117.739998 81.66) (width 0.5) (layer F.Cu) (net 9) (status 20))
 (segment (start 115.999999 69.980001) (end 115.999999 79.920001) (width 0.5) (layer F.Cu) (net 9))
 (segment (start 117.2 68.78) (end 115.999999 69.980001) (width 0.5) (layer F.Cu) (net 9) (status 10))
 (segment (start 133.4 89.7) (end 133.3 89.8) (width 0.5) (layer B.Cu) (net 5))
 (via (at 133.4 89.7) (size 0.8) (drill 0.4) (layers F.Cu B.Cu) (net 5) (status 30))
 (segment (start 135.23599 89.49401) (end 135.07 89.66) (width 0.5) (layer F.Cu) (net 5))
 (segment (start 135.07 89.66) (end 133.32 89.66) (width 0.5) (layer F.Cu) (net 5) (status 20))
 (segment (start 135.23599 77.01501) (end 135.23599 89.49401) (width 0.5) (layer F.Cu) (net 5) (status 10))
 (segment (start 135.382 76.869) (end 135.23599 77.01501) (width 0.5) (layer F.Cu) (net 5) (status 30))
 (segment (start 127.7874 77.0926) (end 126.72 78.16) (width 0.5) (layer F.Cu) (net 14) (status 20))
 (segment (start 127.7874 75.3488) (end 127.7874 77.0926) (width 0.5) (layer F.Cu) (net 14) (status 10))
 (segment (start 125.5268 75.368) (end 124.72 76.1748) (width 0.5) (layer F.Cu) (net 7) (status 10))
 (segment (start 124.72 76.1748) (end 124.72 78.16) (width 0.5) (layer F.Cu) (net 7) (status 20))
 (segment (start 125.5268 75.368) (end 125.5268 75.0443) (width 0.25) (layer F.Cu) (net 7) (status 30))
 (segment (start 120.446201 74.443799) (end 120.396 74.494) (width 0.25) (layer F.Cu) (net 7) (status 30))
 (segment (start 124.926299 74.443799) (end 120.446201 74.443799) (width 0.25) (layer F.Cu) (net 7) (status 20))
 (segment (start 125.5268 75.0443) (end 124.926299 74.443799) (width 0.25) (layer F.Cu) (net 7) (status 10))
 (via (at 131.6 64.6) (size 0.8) (drill 0.4) (layers F.Cu B.Cu) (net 6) (status 30))
 (segment (start 123 62) (end 125.7 62) (width 0.5) (layer F.Cu) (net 6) (status 10))
 (segment (start 125.7 62) (end 129.5 62) (width 0.5) (layer F.Cu) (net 6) (status 20))
 (via (at 125.7 62) (size 0.8) (drill 0.4) (layers F.Cu B.Cu) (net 6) (status 30))
 (segment (start 132.55 66.5) (end 131.2 65.15) (width 0.5) (layer B.Cu) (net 6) (status 30))
 (segment (start 133.4 66.5) (end 132.55 66.5) (width 0.5) (layer B.Cu) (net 6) (status 30))
 (segment (start 129.5 63.45) (end 129.5 62) (width 0.5) (layer B.Cu) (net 6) (status 20))
 (segment (start 131.2 65.15) (end 129.5 63.45) (width 0.5) (layer B.Cu) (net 6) (status 10))
 (segment (start 119.300001 63.899999) (end 119.169999 63.899999) (width 0.5) (layer F.Cu) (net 6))
 (via (at 119.300001 63.899999) (size 0.8) (drill 0.4) (layers F.Cu B.Cu) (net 6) (status 30))
 (segment (start 123 63.415) (end 122.4075 64.0075) (width 0.5) (layer B.Cu) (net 6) (status 20))
 (segment (start 123 62) (end 123 63.415) (width 0.5) (layer B.Cu) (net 6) (status 10))
 (segment (start 122.4075 64.0075) (end 122.385 64.03) (width 0.5) (layer B.Cu) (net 6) (status 30))
 (segment (start 119.407502 64.0075) (end 119.300001 63.899999) (width 0.5) (layer F.Cu) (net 6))
 (segment (start 122.4075 64.0075) (end 122.365 64.0075) (width 0.5) (layer F.Cu) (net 6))
 (segment (start 122.365 64.0075) (end 119.407502 64.0075) (width 0.5) (layer F.Cu) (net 6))
 (via (at 122.365 64.0075) (size 0.5) (drill 0.3) (layers F.Cu B.Cu) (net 6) (status 30))
 (segment (start 130.048 76.832) (end 128.72 78.16) (width 0.5) (layer F.Cu) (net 15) (status 20))
 (segment (start 130.048 75.3488) (end 130.048 76.832) (width 0.5) (layer F.Cu) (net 15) (status 10))
 (via (at 120.2 67.2) (size 0.8) (drill 0.4) (layers F.Cu B.Cu) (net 16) (status 30))
 (segment (start 126.057603 73.993801) (end 122.393801 73.993801) (width 0.25) (layer F.Cu) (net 13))
 (segment (start 126.501801 74.437999) (end 126.057603 73.993801) (width 0.25) (layer F.Cu) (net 13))
 (segment (start 126.501801 76.298001) (end 126.501801 74.437999) (width 0.25) (layer F.Cu) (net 13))
 (segment (start 125.994999 78.690003) (end 125.994999 76.804803) (width 0.25) (layer F.Cu) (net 13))
 (segment (start 125.400001 79.285001) (end 125.994999 78.690003) (width 0.25) (layer F.Cu) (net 13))
 (segment (start 123.845001 79.285001) (end 125.400001 79.285001) (width 0.25) (layer F.Cu) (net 13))
 (segment (start 122.72 78.16) (end 123.845001 79.285001) (width 0.25) (layer F.Cu) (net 13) (status 10))
 (segment (start 125.994999 76.804803) (end 126.501801 76.298001) (width 0.25) (layer F.Cu) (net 13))
 (segment (start 122.393801 73.993801) (end 122.2 73.8) (width 0.25) (layer F.Cu) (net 13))
 (segment (start 122.2 73.8) (end 122.2 70.3) (width 0.25) (layer F.Cu) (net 13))
 (via (at 122.2 70.3) (size 0.8) (drill 0.4) (layers F.Cu B.Cu) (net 13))
 (segment (start 122.2 68.15) (end 122.021 67.971) (width 0.25) (layer B.Cu) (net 13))
 (segment (start 122.2 70.3) (end 122.2 68.15) (width 0.25) (layer B.Cu) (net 13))
 (segment (start 122.021 67.971) (end 121.15 67.1) (width 0.25) (layer B.Cu) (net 13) (status 20))
 (via (at 122.021 67.971) (size 0.5) (drill 0.3) (layers F.Cu B.Cu) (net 13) (status 30))
 (segment (start 126.492 69.9268) (end 123.4 73.0188) (width 0.5) (layer F.Cu) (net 17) (status 20))
 (segment (start 126.492 69.088) (end 126.492 69.9268) (width 0.5) (layer F.Cu) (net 17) (status 10))
 (segment (start 123.4 75.48) (end 120.72 78.16) (width 0.5) (layer F.Cu) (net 12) (status 30))
 (segment (start 123.4 75.4188) (end 123.4 75.48) (width 0.5) (layer F.Cu) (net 12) (status 30))
 (via (at 117.8 62.5) (size 0.8) (drill 0.4) (layers F.Cu B.Cu) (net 18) (status 30))
 (segment (start 123 66.5) (end 129.5 66.5) (width 0.5) (layer F.Cu) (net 11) (status 30))
 (segment (start 120.5 72.6) (end 121.7 72.6) (width 0.5) (layer B.Cu) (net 11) (status 10))
 (segment (start 123 71.3) (end 123 66.5) (width 0.5) (layer B.Cu) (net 11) (status 20))
 (segment (start 121.7 72.6) (end 123 71.3) (width 0.5) (layer B.Cu) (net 11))
 (segment (start 121.15 63.45) (end 121.15 64.5) (width 0.5) (layer B.Cu) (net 11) (status 20))
 (segment (start 120.3 62.6) (end 121.15 63.45) (width 0.5) (layer B.Cu) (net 11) (status 10))
 (segment (start 121.15 64.65) (end 123 66.5) (width 0.5) (layer B.Cu) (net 11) (status 30))
 (segment (start 121.15 64.5) (end 121.15 64.65) (width 0.5) (layer B.Cu) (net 11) (status 30))
 (segment (start 120.550001 65.149999) (end 126.050001 65.149999) (width 0.5) (layer F.Cu) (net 3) (status 10))
 (segment (start 120.3 65.4) (end 120.550001 65.149999) (width 0.5) (layer F.Cu) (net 3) (status 30))
 (segment (start 126.050001 65.149999) (end 127.55 63.65) (width 0.5) (layer F.Cu) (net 3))
 (segment (start 127.55 63.65) (end 127.6 63.6) (width 0.5) (layer F.Cu) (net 3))
 (via (at 127.55 63.65) (size 0.8) (drill 0.4) (layers F.Cu B.Cu) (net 3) (status 30))
 (segment (start 127.65001 63.54999) (end 127.55 63.65) (width 0.5) (layer F.Cu) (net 3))
 (segment (start 134.62501 64.106493) (end 134.068507 63.54999) (width 0.5) (layer F.Cu) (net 3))
 (segment (start 134.62501 70.37149) (end 134.62501 64.106493) (width 0.5) (layer F.Cu) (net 3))
 (segment (start 134.068507 63.54999) (end 127.65001 63.54999) (width 0.5) (layer F.Cu) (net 3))
 (segment (start 133.9375 71.059) (end 134.62501 70.37149) (width 0.5) (layer F.Cu) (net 3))
 (segment (start 131.595802 78.16) (end 130.72 78.16) (width 0.5) (layer F.Cu) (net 1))
 (segment (start 133.357801 76.398001) (end 131.595802 78.16) (width 0.5) (layer F.Cu) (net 1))
 (segment (start 133.357801 75.063197) (end 133.357801 76.398001) (width 0.5) (layer F.Cu) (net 1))
 (segment (start 135.9375 72.483498) (end 133.357801 75.063197) (width 0.5) (layer F.Cu) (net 1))
 (segment (start 135.9375 72.009) (end 135.9375 72.483498) (width 0.5) (layer F.Cu) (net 1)))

